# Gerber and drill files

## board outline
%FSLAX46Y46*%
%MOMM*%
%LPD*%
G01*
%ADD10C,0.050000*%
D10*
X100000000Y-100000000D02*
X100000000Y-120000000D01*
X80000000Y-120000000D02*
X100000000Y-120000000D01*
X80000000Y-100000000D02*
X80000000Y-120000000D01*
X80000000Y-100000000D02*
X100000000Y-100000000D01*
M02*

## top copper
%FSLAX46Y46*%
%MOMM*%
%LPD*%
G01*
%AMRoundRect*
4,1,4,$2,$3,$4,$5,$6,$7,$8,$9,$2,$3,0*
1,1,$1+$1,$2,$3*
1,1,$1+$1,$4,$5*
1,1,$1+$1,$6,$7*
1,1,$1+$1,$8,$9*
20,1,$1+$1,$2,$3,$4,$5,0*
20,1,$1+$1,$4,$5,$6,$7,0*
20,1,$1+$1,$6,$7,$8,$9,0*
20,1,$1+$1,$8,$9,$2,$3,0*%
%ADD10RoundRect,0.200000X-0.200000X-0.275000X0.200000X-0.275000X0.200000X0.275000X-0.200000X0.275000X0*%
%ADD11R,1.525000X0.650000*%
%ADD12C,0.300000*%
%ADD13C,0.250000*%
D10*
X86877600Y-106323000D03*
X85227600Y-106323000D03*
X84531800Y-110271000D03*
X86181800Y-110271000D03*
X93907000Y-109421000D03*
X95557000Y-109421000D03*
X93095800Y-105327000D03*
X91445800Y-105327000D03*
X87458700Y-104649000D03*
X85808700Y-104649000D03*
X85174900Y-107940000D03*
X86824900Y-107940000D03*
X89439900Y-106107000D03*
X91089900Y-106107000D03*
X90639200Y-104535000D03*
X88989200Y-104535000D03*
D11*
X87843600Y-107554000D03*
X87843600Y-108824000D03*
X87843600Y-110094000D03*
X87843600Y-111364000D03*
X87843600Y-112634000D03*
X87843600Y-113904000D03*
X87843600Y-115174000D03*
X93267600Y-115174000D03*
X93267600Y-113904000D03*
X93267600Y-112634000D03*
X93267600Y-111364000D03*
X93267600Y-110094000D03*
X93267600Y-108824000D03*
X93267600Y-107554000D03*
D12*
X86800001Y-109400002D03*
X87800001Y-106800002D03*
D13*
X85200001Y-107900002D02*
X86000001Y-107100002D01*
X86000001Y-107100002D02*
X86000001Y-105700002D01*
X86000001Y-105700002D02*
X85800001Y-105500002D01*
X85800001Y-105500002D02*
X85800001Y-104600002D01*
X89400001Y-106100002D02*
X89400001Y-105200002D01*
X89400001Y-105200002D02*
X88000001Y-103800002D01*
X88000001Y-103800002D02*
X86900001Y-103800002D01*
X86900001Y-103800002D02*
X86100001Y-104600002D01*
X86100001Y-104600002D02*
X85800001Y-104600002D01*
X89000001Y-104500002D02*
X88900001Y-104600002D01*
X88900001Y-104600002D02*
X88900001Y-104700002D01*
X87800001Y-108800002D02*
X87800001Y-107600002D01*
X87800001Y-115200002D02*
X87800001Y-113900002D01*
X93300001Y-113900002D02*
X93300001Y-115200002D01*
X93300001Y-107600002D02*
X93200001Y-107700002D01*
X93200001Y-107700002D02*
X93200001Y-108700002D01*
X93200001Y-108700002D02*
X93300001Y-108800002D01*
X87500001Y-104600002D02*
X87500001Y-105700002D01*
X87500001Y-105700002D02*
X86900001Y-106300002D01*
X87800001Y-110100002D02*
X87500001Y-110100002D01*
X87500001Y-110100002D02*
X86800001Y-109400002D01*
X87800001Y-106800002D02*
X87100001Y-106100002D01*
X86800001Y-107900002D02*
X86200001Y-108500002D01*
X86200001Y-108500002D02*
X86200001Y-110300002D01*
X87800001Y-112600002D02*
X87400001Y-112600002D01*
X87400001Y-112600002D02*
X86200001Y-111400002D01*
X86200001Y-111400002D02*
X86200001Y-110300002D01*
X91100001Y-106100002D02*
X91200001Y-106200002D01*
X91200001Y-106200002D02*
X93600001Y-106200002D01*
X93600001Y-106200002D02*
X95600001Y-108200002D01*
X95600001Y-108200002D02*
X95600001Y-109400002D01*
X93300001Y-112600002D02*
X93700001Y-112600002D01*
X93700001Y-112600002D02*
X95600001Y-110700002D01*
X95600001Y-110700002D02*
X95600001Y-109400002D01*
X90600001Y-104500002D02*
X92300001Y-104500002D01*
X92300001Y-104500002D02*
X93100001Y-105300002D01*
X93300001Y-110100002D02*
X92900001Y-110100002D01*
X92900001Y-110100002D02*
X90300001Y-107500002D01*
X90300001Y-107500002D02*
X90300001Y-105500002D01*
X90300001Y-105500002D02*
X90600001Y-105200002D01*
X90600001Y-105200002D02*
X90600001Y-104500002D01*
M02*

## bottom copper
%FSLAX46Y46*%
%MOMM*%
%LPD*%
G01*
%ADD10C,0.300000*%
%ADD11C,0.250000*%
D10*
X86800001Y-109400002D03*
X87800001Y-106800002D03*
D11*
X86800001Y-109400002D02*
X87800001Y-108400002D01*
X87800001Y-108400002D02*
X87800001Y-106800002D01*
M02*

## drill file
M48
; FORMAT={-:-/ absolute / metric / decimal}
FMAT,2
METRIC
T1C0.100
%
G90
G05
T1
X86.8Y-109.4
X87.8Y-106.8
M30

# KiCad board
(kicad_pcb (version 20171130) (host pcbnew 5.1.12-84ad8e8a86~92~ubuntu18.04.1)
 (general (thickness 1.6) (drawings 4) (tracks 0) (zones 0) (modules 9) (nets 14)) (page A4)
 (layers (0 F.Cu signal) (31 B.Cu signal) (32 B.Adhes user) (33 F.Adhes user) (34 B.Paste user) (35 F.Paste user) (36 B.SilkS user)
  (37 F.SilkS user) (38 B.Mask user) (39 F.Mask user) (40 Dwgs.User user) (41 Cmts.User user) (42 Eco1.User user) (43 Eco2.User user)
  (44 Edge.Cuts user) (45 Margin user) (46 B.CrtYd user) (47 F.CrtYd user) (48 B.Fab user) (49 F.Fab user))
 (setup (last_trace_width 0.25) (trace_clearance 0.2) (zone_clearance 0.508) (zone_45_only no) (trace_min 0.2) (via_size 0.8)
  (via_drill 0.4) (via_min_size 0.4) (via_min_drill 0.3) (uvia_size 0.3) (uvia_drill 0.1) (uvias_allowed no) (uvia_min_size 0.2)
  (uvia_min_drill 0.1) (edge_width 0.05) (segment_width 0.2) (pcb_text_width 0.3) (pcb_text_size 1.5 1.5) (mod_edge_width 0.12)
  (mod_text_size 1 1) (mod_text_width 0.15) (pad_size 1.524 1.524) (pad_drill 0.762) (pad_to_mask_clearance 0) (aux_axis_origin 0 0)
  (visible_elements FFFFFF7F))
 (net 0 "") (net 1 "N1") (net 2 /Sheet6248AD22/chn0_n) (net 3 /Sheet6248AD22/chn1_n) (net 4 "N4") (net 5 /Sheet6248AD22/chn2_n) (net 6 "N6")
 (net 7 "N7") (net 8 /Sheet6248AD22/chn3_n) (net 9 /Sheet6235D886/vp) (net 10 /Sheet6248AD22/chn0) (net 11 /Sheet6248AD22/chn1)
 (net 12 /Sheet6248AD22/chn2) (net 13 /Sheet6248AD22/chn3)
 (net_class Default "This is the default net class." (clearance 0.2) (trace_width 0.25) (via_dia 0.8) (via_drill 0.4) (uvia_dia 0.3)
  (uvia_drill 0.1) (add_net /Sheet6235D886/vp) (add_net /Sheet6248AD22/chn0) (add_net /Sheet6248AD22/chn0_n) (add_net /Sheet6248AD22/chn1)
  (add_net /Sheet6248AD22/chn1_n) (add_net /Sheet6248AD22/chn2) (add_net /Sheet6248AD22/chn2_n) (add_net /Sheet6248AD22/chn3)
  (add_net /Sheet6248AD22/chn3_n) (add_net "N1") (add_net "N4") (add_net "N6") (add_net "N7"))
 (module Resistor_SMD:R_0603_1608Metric (layer F.Cu) (at 86.052600 106.323000)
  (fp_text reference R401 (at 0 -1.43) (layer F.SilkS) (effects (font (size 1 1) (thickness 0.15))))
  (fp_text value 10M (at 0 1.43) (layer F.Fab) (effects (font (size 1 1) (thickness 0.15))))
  (pad 2 smd roundrect (at 0.825 0) (size 0.8 0.95) (layers F.Cu F.Mask F.Paste) (roundrect_rratio 0.25) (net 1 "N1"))
  (pad 1 smd roundrect (at -0.825 0) (size 0.8 0.95) (layers F.Cu F.Mask F.Paste) (roundrect_rratio 0.25) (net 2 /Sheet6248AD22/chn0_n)))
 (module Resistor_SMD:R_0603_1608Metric (layer F.Cu) (at 85.356800 110.271000)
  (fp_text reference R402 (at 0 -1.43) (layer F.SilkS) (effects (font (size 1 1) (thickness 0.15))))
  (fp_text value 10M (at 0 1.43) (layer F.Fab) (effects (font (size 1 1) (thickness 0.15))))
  (pad 1 smd roundrect (at -0.825 0) (size 0.8 0.95) (layers F.Cu F.Mask F.Paste) (roundrect_rratio 0.25) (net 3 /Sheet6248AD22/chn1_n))
  (pad 2 smd roundrect (at 0.825 0) (size 0.8 0.95) (layers F.Cu F.Mask F.Paste) (roundrect_rratio 0.25) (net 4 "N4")))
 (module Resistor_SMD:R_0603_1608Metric (layer F.Cu) (at 94.732000 109.421000)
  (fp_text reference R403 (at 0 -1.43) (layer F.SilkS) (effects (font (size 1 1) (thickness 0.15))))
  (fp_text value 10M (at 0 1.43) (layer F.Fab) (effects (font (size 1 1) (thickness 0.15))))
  (pad 1 smd roundrect (at -0.825 0) (size 0.8 0.95) (layers F.Cu F.Mask F.Paste) (roundrect_rratio 0.25) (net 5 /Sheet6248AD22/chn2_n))
  (pad 2 smd roundrect (at 0.825 0) (size 0.8 0.95) (layers F.Cu F.Mask F.Paste) (roundrect_rratio 0.25) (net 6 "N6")))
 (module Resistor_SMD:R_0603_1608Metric (layer F.Cu) (at 92.270800 105.327000)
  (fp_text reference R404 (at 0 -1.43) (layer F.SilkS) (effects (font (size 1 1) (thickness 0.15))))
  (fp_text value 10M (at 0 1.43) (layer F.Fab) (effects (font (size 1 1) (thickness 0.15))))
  (pad 2 smd roundrect (at 0.825 0) (size 0.8 0.95) (layers F.Cu F.Mask F.Paste) (roundrect_rratio 0.25) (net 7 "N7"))
  (pad 1 smd roundrect (at -0.825 0) (size 0.8 0.95) (layers F.Cu F.Mask F.Paste) (roundrect_rratio 0.25) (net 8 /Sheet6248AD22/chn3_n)))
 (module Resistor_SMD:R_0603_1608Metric (layer F.Cu) (at 86.633700 104.649000)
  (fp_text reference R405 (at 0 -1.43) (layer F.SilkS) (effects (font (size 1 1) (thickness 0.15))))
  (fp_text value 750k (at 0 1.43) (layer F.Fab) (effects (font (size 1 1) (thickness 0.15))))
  (pad 2 smd roundrect (at 0.825 0) (size 0.8 0.95) (layers F.Cu F.Mask F.Paste) (roundrect_rratio 0.25) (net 1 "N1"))
  (pad 1 smd roundrect (at -0.825 0) (size 0.8 0.95) (layers F.Cu F.Mask F.Paste) (roundrect_rratio 0.25) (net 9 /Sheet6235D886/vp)))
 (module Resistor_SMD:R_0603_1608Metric (layer F.Cu) (at 85.999900 107.940000)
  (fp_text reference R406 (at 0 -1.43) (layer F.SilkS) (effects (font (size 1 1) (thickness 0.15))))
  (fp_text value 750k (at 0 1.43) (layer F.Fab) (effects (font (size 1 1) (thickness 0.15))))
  (pad 1 smd roundrect (at -0.825 0) (size 0.8 0.95) (layers F.Cu F.Mask F.Paste) (roundrect_rratio 0.25) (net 9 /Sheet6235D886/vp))
  (pad 2 smd roundrect (at 0.825 0) (size 0.8 0.95) (layers F.Cu F.Mask F.Paste) (roundrect_rratio 0.25) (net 4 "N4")))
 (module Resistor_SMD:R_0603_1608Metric (layer F.Cu) (at 90.264900 106.107000)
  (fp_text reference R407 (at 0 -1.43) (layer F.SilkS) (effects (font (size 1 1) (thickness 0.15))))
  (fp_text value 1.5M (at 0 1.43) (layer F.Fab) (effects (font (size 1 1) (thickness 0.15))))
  (pad 1 smd roundrect (at -0.825 0) (size 0.8 0.95) (layers F.Cu F.Mask F.Paste) (roundrect_rratio 0.25) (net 9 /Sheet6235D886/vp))
  (pad 2 smd roundrect (at 0.825 0) (size 0.8 0.95) (layers F.Cu F.Mask F.Paste) (roundrect_rratio 0.25) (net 6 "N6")))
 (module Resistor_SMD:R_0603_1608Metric (layer F.Cu) (at 89.814200 104.535000)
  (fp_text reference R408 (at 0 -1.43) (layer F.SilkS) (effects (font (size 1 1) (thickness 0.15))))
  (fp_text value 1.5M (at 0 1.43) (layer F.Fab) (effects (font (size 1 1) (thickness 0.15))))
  (pad 2 smd roundrect (at 0.825 0) (size 0.8 0.95) (layers F.Cu F.Mask F.Paste) (roundrect_rratio 0.25) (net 7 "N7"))
  (pad 1 smd roundrect (at -0.825 0) (size 0.8 0.95) (layers F.Cu F.Mask F.Paste) (roundrect_rratio 0.25) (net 9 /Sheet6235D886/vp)))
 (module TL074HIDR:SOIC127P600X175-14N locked (layer F.Cu) (at 90.555600 111.364000)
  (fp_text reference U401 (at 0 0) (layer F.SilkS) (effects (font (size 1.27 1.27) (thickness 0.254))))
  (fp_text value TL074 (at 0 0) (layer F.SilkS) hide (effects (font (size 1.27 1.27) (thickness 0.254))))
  (pad 1 smd rect (at -2.712 -3.81 90.000000) (size 0.65 1.525) (layers F.Cu F.Mask F.Paste) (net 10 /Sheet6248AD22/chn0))
  (pad 2 smd rect (at -2.712 -2.54 90.000000) (size 0.65 1.525) (layers F.Cu F.Mask F.Paste) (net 10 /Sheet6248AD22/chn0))
  (pad 3 smd rect (at -2.712 -1.27 90.000000) (size 0.65 1.525) (layers F.Cu F.Mask F.Paste) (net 1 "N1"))
  (pad 4 smd rect (at -2.712 0 90.000000) (size 0.65 1.525) (layers F.Cu F.Mask F.Paste))
  (pad 5 smd rect (at -2.712 1.27 90.000000) (size 0.65 1.525) (layers F.Cu F.Mask F.Paste) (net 4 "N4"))
  (pad 6 smd rect (at -2.712 2.54 90.000000) (size 0.65 1.525) (layers F.Cu F.Mask F.Paste) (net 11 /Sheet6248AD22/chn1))
  (pad 7 smd rect (at -2.712 3.81 90.000000) (size 0.65 1.525) (layers F.Cu F.Mask F.Paste) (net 11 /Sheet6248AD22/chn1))
  (pad 8 smd rect (at 2.712 3.81 90.000000) (size 0.65 1.525) (layers F.Cu F.Mask F.Paste) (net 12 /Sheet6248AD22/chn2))
  (pad 9 smd rect (at 2.712 2.54 90.000000) (size 0.65 1.525) (layers F.Cu F.Mask F.Paste) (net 12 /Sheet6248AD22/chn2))
  (pad 10 smd rect (at 2.712 1.27 90.000000) (size 0.65 1.525) (layers F.Cu F.Mask F.Paste) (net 6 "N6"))
  (pad 11 smd rect (at 2.712 0 90.000000) (size 0.65 1.525) (layers F.Cu F.Mask F.Paste))
  (pad 12 smd rect (at 2.712 -1.27 90.000000) (size 0.65 1.525) (layers F.Cu F.Mask F.Paste) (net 7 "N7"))
  (pad 13 smd rect (at 2.712 -2.54 90.000000) (size 0.65 1.525) (layers F.Cu F.Mask F.Paste) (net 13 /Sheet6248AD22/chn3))
  (pad 14 smd rect (at 2.712 -3.81 90.000000) (size 0.65 1.525) (layers F.Cu F.Mask F.Paste) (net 13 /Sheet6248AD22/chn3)))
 (gr_line (start 100 100) (end 100 120) (layer Edge.Cuts) (width 0.05))
 (gr_line (start 80 120) (end 100 120) (layer Edge.Cuts) (width 0.05))
 (gr_line (start 80 100) (end 80 120) (layer Edge.Cuts) (width 0.05))
 (gr_line (start 80 100) (end 100 100) (layer Edge.Cuts) (width 0.05))
 (segment (start 85.200001 107.900002) (end 86.000001 107.100002) (width 0.250000) (layer F.Cu) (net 9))
 (segment (start 86.000001 107.100002) (end 86.000001 105.700002) (width 0.250000) (layer F.Cu) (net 9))
 (segment (start 86.000001 105.700002) (end 85.800001 105.500002) (width 0.250000) (layer F.Cu) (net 9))
 (segment (start 85.800001 105.500002) (end 85.800001 104.600002) (width 0.250000) (layer F.Cu) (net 9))
 (segment (start 89.400001 106.100002) (end 89.400001 105.200002) (width 0.250000) (layer F.Cu) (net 9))
 (segment (start 89.400001 105.200002) (end 88.000001 103.800002) (width 0.250000) (layer F.Cu) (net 9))
 (segment (start 88.000001 103.800002) (end 86.900001 103.800002) (width 0.250000) (layer F.Cu) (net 9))
 (segment (start 86.900001 103.800002) (end 86.100001 104.600002) (width 0.250000) (layer F.Cu) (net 9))
 (segment (start 86.100001 104.600002) (end 85.800001 104.600002) (width 0.250000) (layer F.Cu) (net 9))
 (segment (start 89.000001 104.500002) (end 88.900001 104.600002) (width 0.250000) (layer F.Cu) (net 9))
 (segment (start 88.900001 104.600002) (end 88.900001 104.700002) (width 0.250000) (layer F.Cu) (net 9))
 (segment (start 87.800001 108.800002) (end 87.800001 107.600002) (width 0.250000) (layer F.Cu) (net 10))
 (segment (start 87.800001 115.200002) (end 87.800001 113.900002) (width 0.250000) (layer F.Cu) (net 11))
 (segment (start 93.300001 113.900002) (end 93.300001 115.200002) (width 0.250000) (layer F.Cu) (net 12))
 (segment (start 93.300001 107.600002) (end 93.200001 107.700002) (width 0.250000) (layer F.Cu) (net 13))
 (segment (start 93.200001 107.700002) (end 93.200001 108.700002) (width 0.250000) (layer F.Cu) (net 13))
 (segment (start 93.200001 108.700002) (end 93.300001 108.800002) (width 0.250000) (layer F.Cu) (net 13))
 (segment (start 87.500001 104.600002) (end 87.500001 105.700002) (width 0.250000) (layer F.Cu) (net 1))
 (segment (start 87.500001 105.700002) (end 86.900001 106.300002) (width 0.250000) (layer F.Cu) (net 1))
 (segment (start 87.800001 110.100002) (end 87.500001 110.100002) (width 0.250000) (layer F.Cu) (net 1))
 (segment (start 87.500001 110.100002) (end 86.800001 109.400002) (width 0.250000) (layer F.Cu) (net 1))
 (segment (start 86.800001 109.400002) (end 87.800001 108.400002) (width 0.250000) (layer B.Cu) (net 1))
 (segment (start 87.800001 108.400002) (end 87.800001 106.800002) (width 0.250000) (layer B.Cu) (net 1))
 (segment (start 87.800001 106.800002) (end 87.100001 106.100002) (width 0.250000) (layer F.Cu) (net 1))
 (via micro (at 86.800001 109.400002) (size 0.300000) (drill 0.100000) (layers F.Cu B.Cu) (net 1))
 (via micro (at 87.800001 106.800002) (size 0.300000) (drill 0.100000) (layers F.Cu B.Cu) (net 1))
 (segment (start 86.800001 107.900002) (end 86.200001 108.500002) (width 0.250000) (layer F.Cu) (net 4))
 (segment (start 86.200001 108.500002) (end 86.200001 110.300002) (width 0.250000) (layer F.Cu) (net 4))
 (segment (start 87.800001 112.600002) (end 87.400001 112.600002) (width 0.250000) (layer F.Cu) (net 4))
 (segment (start 87.400001 112.600002) (end 86.200001 111.400002) (width 0.250000) (layer F.Cu) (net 4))
 (segment (start 86.200001 111.400002) (end 86.200001 110.300002) (width 0.250000) (layer F.Cu) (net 4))
 (segment (start 91.100001 106.100002) (end 91.200001 106.200002) (width 0.250000) (layer F.Cu) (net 6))
 (segment (start 91.200001 106.200002) (end 93.600001 106.200002) (width 0.250000) (layer F.Cu) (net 6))
 (segment (start 93.600001 106.200002) (end 95.600001 108.200002) (width 0.250000) (layer F.Cu) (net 6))
 (segment (start 95.600001 108.200002) (end 95.600001 109.400002) (width 0.250000) (layer F.Cu) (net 6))
 (segment (start 93.300001 112.600002) (end 93.700001 112.600002) (width 0.250000) (layer F.Cu) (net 6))
 (segment (start 93.700001 112.600002) (end 95.600001 110.700002) (width 0.250000) (layer F.Cu) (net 6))
 (segment (start 95.600001 110.700002) (end 95.600001 109.400002) (width 0.250000) (layer F.Cu) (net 6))
 (segment (start 90.600001 104.500002) (end 92.300001 104.500002) (width 0.250000) (layer F.Cu) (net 7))
 (segment (start 92.300001 104.500002) (end 93.100001 105.300002) (width 0.250000) (layer F.Cu) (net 7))
 (segment (start 93.300001 110.100002) (end 92.900001 110.100002) (width 0.250000) (layer F.Cu) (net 7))
 (segment (start 92.900001 110.100002) (end 90.300001 107.500002) (width 0.250000) (layer F.Cu) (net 7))
 (segment (start 90.300001 107.500002) (end 90.300001 105.500002) (width 0.250000) (layer F.Cu) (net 7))
 (segment (start 90.300001 105.500002) (end 90.600001 105.200002) (width 0.250000) (layer F.Cu) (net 7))
 (segment (start 90.600001 105.200002) (end 90.600001 104.500002) (width 0.250000) (layer F.Cu) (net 7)))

